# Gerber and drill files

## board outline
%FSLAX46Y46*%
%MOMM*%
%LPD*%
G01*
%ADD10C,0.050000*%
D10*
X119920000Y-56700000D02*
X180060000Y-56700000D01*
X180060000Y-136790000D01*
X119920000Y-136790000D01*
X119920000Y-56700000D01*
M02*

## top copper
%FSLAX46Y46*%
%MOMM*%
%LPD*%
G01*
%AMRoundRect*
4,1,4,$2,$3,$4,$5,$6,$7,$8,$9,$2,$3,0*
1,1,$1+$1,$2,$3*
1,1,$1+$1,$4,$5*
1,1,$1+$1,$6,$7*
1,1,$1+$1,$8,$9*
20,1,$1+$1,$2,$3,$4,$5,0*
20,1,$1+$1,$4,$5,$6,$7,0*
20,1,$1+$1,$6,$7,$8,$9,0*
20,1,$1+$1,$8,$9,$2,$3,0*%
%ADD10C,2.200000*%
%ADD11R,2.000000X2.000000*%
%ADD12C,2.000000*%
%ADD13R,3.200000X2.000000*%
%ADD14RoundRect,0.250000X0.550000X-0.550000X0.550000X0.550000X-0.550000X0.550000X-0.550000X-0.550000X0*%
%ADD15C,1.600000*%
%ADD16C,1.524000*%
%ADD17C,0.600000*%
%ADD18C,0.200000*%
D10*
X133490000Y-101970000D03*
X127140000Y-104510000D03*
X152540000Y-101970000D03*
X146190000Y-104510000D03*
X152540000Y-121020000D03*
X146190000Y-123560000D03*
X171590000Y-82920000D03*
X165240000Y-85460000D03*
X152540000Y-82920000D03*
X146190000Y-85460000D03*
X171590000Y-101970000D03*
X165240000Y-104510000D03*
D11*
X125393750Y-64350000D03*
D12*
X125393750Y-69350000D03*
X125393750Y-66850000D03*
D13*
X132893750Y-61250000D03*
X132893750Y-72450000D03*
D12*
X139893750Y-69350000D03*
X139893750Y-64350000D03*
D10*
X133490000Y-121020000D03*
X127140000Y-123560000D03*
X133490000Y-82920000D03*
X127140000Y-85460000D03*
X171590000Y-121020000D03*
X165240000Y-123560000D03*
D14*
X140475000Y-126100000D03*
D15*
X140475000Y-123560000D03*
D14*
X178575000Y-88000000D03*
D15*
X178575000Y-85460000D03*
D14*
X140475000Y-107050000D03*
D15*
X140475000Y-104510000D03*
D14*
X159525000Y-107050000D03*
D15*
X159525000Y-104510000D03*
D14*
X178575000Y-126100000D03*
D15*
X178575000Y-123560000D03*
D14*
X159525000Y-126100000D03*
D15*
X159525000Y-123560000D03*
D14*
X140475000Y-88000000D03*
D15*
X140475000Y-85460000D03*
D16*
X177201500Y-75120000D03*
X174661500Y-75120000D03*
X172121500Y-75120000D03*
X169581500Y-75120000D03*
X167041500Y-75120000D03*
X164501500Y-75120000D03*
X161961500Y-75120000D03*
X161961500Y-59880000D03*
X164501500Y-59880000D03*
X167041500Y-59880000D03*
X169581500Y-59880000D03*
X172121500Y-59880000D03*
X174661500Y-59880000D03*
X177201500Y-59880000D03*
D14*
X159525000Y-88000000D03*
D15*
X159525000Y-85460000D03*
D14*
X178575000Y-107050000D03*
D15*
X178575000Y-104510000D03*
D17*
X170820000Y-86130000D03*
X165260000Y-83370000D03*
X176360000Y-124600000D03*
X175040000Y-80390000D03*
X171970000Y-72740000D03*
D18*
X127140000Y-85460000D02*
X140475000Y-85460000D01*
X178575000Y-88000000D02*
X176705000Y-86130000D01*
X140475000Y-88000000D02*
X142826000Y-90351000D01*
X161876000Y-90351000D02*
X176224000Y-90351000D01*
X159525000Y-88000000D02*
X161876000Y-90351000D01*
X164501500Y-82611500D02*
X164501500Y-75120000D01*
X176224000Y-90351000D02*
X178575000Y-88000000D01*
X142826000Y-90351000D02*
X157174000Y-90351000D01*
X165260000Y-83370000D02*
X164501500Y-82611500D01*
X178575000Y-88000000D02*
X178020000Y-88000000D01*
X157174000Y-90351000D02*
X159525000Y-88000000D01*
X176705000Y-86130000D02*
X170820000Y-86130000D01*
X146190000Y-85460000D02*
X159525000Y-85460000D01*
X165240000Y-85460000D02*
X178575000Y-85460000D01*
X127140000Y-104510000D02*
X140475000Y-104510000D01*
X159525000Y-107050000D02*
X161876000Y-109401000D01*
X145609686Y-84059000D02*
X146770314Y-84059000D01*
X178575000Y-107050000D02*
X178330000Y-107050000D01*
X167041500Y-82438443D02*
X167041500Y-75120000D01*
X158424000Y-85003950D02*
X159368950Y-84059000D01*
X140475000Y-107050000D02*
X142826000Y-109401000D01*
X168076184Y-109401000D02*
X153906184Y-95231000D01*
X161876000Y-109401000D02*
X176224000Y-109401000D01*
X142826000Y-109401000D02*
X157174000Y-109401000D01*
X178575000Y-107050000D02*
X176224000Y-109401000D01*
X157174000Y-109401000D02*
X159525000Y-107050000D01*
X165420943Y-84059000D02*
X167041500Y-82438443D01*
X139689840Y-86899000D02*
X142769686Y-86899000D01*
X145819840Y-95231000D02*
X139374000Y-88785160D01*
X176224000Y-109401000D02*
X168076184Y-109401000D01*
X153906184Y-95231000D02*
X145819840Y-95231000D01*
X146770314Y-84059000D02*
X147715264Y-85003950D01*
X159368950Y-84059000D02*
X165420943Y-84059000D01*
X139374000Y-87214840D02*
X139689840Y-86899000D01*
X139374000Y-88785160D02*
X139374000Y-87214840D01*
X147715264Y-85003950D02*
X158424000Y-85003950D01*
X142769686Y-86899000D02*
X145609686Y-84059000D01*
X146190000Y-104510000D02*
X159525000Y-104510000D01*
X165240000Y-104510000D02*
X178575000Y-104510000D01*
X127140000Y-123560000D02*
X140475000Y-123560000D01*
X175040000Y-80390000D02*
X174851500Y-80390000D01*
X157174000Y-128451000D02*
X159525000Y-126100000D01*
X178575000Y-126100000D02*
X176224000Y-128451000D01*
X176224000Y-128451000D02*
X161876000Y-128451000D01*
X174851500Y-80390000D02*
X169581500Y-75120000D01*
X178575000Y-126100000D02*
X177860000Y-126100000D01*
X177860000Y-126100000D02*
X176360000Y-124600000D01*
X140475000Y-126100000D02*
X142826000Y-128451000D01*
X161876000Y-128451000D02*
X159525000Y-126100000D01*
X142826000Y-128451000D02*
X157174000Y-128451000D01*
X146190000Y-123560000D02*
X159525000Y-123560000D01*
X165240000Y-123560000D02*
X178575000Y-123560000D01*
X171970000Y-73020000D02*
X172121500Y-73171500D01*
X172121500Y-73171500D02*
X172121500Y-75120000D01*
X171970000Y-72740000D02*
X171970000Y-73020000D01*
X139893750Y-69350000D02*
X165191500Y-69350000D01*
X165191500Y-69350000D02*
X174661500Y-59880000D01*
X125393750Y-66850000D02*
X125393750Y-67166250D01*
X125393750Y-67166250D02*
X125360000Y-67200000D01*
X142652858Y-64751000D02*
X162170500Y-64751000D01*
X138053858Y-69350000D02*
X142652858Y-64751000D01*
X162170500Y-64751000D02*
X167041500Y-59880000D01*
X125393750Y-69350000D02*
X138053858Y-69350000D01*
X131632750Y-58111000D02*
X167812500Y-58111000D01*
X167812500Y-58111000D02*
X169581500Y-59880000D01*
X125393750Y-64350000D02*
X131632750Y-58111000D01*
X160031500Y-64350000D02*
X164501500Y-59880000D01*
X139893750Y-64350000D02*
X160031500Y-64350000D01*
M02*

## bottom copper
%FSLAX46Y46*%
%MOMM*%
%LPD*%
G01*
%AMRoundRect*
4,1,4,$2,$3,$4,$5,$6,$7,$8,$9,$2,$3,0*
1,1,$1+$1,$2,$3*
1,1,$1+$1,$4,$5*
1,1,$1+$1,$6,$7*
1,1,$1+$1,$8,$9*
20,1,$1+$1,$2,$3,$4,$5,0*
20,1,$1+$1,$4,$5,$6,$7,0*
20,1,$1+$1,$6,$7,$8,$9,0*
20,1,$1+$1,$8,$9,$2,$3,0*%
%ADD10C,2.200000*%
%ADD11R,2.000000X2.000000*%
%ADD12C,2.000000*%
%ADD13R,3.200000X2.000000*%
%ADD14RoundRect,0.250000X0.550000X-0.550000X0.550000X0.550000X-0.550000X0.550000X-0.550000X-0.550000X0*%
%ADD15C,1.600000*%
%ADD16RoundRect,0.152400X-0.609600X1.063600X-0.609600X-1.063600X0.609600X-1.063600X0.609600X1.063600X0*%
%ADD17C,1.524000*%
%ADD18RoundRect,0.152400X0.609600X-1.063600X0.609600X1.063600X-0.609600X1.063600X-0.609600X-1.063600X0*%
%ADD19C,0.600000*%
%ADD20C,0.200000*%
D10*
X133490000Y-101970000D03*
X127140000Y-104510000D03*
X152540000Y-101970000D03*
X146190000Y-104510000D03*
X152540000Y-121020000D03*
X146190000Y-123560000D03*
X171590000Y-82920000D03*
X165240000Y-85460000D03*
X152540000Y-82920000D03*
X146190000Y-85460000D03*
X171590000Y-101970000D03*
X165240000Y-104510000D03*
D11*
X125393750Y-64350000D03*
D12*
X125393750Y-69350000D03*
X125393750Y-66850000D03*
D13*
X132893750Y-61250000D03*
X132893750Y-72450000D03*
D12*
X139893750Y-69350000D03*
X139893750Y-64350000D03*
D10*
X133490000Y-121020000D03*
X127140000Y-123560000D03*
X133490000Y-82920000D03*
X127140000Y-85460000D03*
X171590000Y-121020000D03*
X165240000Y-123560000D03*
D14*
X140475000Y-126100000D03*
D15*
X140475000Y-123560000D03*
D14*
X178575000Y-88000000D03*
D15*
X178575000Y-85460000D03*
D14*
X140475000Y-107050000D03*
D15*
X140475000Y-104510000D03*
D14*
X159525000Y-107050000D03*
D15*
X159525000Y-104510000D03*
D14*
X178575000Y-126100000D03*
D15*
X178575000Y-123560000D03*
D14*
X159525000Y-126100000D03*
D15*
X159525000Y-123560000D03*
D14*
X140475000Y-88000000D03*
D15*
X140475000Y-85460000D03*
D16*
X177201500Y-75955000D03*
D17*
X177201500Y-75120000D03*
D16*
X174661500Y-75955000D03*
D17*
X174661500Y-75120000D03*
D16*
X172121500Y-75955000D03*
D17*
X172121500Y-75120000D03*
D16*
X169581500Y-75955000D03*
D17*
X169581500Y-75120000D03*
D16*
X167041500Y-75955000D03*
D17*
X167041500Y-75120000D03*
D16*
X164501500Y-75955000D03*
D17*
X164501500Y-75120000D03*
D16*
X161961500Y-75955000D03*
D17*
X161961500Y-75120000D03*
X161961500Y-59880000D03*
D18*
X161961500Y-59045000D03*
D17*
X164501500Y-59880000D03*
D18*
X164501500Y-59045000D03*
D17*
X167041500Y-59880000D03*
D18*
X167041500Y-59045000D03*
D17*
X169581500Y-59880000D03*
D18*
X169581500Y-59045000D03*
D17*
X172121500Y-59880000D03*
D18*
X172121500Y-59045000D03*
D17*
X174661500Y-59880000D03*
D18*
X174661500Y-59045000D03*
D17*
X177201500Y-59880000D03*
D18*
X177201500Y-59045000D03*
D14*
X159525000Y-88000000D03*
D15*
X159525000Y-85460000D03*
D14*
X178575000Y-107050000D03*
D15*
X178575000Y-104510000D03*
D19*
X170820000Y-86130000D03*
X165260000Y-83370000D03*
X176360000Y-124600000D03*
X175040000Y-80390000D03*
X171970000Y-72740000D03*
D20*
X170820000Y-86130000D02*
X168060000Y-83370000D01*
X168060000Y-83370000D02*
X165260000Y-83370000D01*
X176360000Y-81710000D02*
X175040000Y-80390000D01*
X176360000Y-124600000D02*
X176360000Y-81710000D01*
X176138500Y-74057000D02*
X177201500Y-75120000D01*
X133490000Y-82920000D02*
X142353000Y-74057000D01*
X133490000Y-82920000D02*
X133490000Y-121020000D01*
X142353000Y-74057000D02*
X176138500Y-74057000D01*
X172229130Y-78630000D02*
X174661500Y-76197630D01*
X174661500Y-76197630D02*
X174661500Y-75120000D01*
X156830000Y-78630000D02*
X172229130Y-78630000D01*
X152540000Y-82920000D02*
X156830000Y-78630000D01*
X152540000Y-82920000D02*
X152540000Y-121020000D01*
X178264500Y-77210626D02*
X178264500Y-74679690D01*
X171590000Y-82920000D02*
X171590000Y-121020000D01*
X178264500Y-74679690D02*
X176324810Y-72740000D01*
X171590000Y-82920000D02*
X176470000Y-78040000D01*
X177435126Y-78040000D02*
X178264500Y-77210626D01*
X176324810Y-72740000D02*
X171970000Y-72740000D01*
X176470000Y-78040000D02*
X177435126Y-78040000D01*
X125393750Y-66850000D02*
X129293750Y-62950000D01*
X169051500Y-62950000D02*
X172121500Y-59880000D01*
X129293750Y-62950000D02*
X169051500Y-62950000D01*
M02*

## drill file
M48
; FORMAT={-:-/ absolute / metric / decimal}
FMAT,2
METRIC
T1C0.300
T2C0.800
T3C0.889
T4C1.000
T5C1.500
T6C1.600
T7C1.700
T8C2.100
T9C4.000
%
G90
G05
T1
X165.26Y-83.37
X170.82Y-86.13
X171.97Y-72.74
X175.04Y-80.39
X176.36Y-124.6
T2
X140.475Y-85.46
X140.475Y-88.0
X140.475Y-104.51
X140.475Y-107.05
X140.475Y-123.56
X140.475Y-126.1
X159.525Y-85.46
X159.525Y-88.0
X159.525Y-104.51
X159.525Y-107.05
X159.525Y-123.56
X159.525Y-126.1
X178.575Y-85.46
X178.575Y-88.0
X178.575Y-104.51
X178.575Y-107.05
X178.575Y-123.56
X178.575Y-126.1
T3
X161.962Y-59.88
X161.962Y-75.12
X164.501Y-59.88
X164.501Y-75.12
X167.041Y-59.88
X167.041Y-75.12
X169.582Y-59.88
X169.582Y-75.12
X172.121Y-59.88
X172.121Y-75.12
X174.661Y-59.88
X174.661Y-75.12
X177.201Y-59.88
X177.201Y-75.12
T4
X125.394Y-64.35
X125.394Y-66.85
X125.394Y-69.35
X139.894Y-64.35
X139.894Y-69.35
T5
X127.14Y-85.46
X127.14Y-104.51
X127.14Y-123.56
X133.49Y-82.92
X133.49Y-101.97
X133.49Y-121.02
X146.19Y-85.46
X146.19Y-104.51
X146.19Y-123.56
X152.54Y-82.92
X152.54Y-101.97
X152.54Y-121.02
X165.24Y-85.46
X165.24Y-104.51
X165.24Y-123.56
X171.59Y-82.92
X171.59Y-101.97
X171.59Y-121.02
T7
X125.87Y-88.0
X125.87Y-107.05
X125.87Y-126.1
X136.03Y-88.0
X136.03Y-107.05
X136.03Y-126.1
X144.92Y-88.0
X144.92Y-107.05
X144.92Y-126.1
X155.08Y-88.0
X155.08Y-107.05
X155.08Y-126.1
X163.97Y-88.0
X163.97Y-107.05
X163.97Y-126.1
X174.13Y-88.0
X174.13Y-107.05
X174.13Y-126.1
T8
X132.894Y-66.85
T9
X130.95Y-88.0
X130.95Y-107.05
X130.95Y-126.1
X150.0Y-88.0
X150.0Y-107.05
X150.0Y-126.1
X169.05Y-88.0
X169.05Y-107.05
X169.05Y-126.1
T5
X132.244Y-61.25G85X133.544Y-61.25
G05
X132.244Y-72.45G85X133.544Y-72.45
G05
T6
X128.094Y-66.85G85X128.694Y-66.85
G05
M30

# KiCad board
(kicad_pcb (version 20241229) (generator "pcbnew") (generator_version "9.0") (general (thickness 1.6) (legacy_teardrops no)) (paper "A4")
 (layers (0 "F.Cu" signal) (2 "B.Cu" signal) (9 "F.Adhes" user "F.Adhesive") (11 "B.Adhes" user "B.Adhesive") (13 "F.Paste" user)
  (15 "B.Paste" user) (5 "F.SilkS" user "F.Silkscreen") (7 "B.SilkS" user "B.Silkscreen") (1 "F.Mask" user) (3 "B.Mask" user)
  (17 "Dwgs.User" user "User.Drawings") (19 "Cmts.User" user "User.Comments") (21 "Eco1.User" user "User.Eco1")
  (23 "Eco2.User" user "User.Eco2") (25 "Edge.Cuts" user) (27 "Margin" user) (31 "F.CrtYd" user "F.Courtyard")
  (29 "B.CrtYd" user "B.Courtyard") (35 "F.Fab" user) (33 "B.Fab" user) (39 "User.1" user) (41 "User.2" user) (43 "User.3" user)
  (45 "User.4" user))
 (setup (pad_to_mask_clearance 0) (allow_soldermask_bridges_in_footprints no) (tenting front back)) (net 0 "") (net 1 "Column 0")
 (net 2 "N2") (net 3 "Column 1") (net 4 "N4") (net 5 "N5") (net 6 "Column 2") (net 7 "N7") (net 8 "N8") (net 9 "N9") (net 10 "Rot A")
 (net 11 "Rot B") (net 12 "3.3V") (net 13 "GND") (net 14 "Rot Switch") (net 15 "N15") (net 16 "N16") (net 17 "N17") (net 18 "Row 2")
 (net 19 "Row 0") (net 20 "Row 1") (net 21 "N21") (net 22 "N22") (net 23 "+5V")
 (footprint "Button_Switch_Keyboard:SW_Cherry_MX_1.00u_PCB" (layer "F.Cu") (at 133.49 101.97)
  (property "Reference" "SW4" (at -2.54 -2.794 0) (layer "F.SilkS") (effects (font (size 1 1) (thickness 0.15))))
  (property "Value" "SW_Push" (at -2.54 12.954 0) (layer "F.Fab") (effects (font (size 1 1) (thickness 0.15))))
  (pad "" np_thru_hole circle (at -7.62 5.08) (size 1.7 1.7) (drill 1.7) (layers "*.Cu" "*.Mask"))
  (pad "" np_thru_hole circle (at -2.54 5.08) (size 4 4) (drill 4) (layers "*.Cu" "*.Mask"))
  (pad "" np_thru_hole circle (at 2.54 5.08) (size 1.7 1.7) (drill 1.7) (layers "*.Cu" "*.Mask"))
  (pad "1" thru_hole circle (at 0 0) (size 2.2 2.2) (drill 1.5) (layers "*.Cu" "*.Mask") (remove_unused_layers no) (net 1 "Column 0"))
  (pad "2" thru_hole circle (at -6.35 2.54) (size 2.2 2.2) (drill 1.5) (layers "*.Cu" "*.Mask") (remove_unused_layers no) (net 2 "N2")))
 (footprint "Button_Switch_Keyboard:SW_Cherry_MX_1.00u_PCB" (layer "F.Cu") (at 152.54 101.97)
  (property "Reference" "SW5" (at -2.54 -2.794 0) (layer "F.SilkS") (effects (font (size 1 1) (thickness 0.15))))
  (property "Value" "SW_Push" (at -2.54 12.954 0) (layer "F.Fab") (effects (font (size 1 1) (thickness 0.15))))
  (pad "" np_thru_hole circle (at -7.62 5.08) (size 1.7 1.7) (drill 1.7) (layers "*.Cu" "*.Mask"))
  (pad "" np_thru_hole circle (at -2.54 5.08) (size 4 4) (drill 4) (layers "*.Cu" "*.Mask"))
  (pad "" np_thru_hole circle (at 2.54 5.08) (size 1.7 1.7) (drill 1.7) (layers "*.Cu" "*.Mask"))
  (pad "1" thru_hole circle (at 0 0) (size 2.2 2.2) (drill 1.5) (layers "*.Cu" "*.Mask") (remove_unused_layers no) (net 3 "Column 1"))
  (pad "2" thru_hole circle (at -6.35 2.54) (size 2.2 2.2) (drill 1.5) (layers "*.Cu" "*.Mask") (remove_unused_layers no) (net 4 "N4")))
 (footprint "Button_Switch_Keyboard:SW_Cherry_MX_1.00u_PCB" (layer "F.Cu") (at 152.54 121.02)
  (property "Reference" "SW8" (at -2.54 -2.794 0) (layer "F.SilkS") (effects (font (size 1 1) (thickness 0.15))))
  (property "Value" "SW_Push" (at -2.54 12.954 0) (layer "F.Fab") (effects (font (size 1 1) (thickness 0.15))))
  (pad "" np_thru_hole circle (at -7.62 5.08) (size 1.7 1.7) (drill 1.7) (layers "*.Cu" "*.Mask"))
  (pad "" np_thru_hole circle (at -2.54 5.08) (size 4 4) (drill 4) (layers "*.Cu" "*.Mask"))
  (pad "" np_thru_hole circle (at 2.54 5.08) (size 1.7 1.7) (drill 1.7) (layers "*.Cu" "*.Mask"))
  (pad "1" thru_hole circle (at 0 0) (size 2.2 2.2) (drill 1.5) (layers "*.Cu" "*.Mask") (remove_unused_layers no) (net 3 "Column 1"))
  (pad "2" thru_hole circle (at -6.35 2.54) (size 2.2 2.2) (drill 1.5) (layers "*.Cu" "*.Mask") (remove_unused_layers no) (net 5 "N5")))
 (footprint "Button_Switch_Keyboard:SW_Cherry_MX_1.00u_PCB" (layer "F.Cu") (at 171.59 82.92)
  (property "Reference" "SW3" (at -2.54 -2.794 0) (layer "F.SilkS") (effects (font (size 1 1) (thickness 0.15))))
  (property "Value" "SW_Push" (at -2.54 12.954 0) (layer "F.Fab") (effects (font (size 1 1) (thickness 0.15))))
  (pad "" np_thru_hole circle (at -7.62 5.08) (size 1.7 1.7) (drill 1.7) (layers "*.Cu" "*.Mask"))
  (pad "" np_thru_hole circle (at -2.54 5.08) (size 4 4) (drill 4) (layers "*.Cu" "*.Mask"))
  (pad "" np_thru_hole circle (at 2.54 5.08) (size 1.7 1.7) (drill 1.7) (layers "*.Cu" "*.Mask"))
  (pad "1" thru_hole circle (at 0 0) (size 2.2 2.2) (drill 1.5) (layers "*.Cu" "*.Mask") (remove_unused_layers no) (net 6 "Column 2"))
  (pad "2" thru_hole circle (at -6.35 2.54) (size 2.2 2.2) (drill 1.5) (layers "*.Cu" "*.Mask") (remove_unused_layers no) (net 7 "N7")))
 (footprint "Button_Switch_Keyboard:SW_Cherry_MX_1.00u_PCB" (layer "F.Cu") (at 152.54 82.92)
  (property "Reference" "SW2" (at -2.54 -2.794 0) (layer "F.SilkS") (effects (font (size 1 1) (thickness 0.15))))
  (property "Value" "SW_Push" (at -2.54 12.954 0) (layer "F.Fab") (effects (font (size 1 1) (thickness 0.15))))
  (pad "" np_thru_hole circle (at -7.62 5.08) (size 1.7 1.7) (drill 1.7) (layers "*.Cu" "*.Mask"))
  (pad "" np_thru_hole circle (at -2.54 5.08) (size 4 4) (drill 4) (layers "*.Cu" "*.Mask"))
  (pad "" np_thru_hole circle (at 2.54 5.08) (size 1.7 1.7) (drill 1.7) (layers "*.Cu" "*.Mask"))
  (pad "1" thru_hole circle (at 0 0) (size 2.2 2.2) (drill 1.5) (layers "*.Cu" "*.Mask") (remove_unused_layers no) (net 3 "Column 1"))
  (pad "2" thru_hole circle (at -6.35 2.54) (size 2.2 2.2) (drill 1.5) (layers "*.Cu" "*.Mask") (remove_unused_layers no) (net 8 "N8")))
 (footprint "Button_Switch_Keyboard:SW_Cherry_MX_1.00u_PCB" (layer "F.Cu") (at 171.59 101.97)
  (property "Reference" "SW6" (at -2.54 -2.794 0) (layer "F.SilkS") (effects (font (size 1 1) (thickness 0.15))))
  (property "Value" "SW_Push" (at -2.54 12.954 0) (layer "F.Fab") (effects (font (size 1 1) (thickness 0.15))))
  (pad "" np_thru_hole circle (at -7.62 5.08) (size 1.7 1.7) (drill 1.7) (layers "*.Cu" "*.Mask"))
  (pad "" np_thru_hole circle (at -2.54 5.08) (size 4 4) (drill 4) (layers "*.Cu" "*.Mask"))
  (pad "" np_thru_hole circle (at 2.54 5.08) (size 1.7 1.7) (drill 1.7) (layers "*.Cu" "*.Mask"))
  (pad "1" thru_hole circle (at 0 0) (size 2.2 2.2) (drill 1.5) (layers "*.Cu" "*.Mask") (remove_unused_layers no) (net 6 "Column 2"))
  (pad "2" thru_hole circle (at -6.35 2.54) (size 2.2 2.2) (drill 1.5) (layers "*.Cu" "*.Mask") (remove_unused_layers no) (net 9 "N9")))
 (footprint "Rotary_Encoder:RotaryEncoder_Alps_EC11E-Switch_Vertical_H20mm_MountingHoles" (layer "F.Cu") (at 125.39375 64.35)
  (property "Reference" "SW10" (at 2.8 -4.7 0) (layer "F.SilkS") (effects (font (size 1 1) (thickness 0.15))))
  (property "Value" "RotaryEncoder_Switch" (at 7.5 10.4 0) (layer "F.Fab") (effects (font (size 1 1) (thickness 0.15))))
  (pad "" np_thru_hole oval (at 3 2.5) (size 2.2 1.6) (drill oval 2.2 1.6) (layers "*.Mask"))
  (pad "" np_thru_hole circle (at 7.5 2.5) (size 2.1 2.1) (drill 2.1) (layers "*.Mask"))
  (pad "A" thru_hole rect (at 0 0) (size 2 2) (drill 1) (layers "*.Cu" "*.Mask") (remove_unused_layers no) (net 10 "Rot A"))
  (pad "B" thru_hole circle (at 0 5) (size 2 2) (drill 1) (layers "*.Cu" "*.Mask") (remove_unused_layers no) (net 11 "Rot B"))
  (pad "C" thru_hole circle (at 0 2.5) (size 2 2) (drill 1) (layers "*.Cu" "*.Mask") (remove_unused_layers no) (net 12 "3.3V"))
  (pad "MP" thru_hole rect (at 7.5 -3.1) (size 3.2 2) (drill oval 2.8 1.5) (layers "*.Cu" "*.Mask") (remove_unused_layers no))
  (pad "MP" thru_hole rect (at 7.5 8.1) (size 3.2 2) (drill oval 2.8 1.5) (layers "*.Cu" "*.Mask") (remove_unused_layers no))
  (pad "S1" thru_hole circle (at 14.5 5) (size 2 2) (drill 1) (layers "*.Cu" "*.Mask") (remove_unused_layers no) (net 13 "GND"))
  (pad "S2" thru_hole circle (at 14.5 0) (size 2 2) (drill 1) (layers "*.Cu" "*.Mask") (remove_unused_layers no) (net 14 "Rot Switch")))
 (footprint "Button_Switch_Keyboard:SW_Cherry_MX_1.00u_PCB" (layer "F.Cu") (at 133.49 121.02)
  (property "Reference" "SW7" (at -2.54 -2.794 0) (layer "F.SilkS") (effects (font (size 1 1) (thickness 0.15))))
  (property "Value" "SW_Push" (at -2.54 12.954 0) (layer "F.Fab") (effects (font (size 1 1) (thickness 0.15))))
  (pad "" np_thru_hole circle (at -7.62 5.08) (size 1.7 1.7) (drill 1.7) (layers "*.Cu" "*.Mask"))
  (pad "" np_thru_hole circle (at -2.54 5.08) (size 4 4) (drill 4) (layers "*.Cu" "*.Mask"))
  (pad "" np_thru_hole circle (at 2.54 5.08) (size 1.7 1.7) (drill 1.7) (layers "*.Cu" "*.Mask"))
  (pad "1" thru_hole circle (at 0 0) (size 2.2 2.2) (drill 1.5) (layers "*.Cu" "*.Mask") (remove_unused_layers no) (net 1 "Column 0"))
  (pad "2" thru_hole circle (at -6.35 2.54) (size 2.2 2.2) (drill 1.5) (layers "*.Cu" "*.Mask") (remove_unused_layers no) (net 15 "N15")))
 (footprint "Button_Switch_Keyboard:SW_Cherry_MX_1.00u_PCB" (layer "F.Cu") (at 133.49 82.92)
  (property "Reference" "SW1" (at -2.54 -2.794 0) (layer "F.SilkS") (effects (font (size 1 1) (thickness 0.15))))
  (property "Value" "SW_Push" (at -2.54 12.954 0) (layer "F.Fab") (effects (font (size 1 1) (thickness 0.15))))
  (pad "" np_thru_hole circle (at -7.62 5.08) (size 1.7 1.7) (drill 1.7) (layers "*.Cu" "*.Mask"))
  (pad "" np_thru_hole circle (at -2.54 5.08) (size 4 4) (drill 4) (layers "*.Cu" "*.Mask"))
  (pad "" np_thru_hole circle (at 2.54 5.08) (size 1.7 1.7) (drill 1.7) (layers "*.Cu" "*.Mask"))
  (pad "1" thru_hole circle (at 0 0) (size 2.2 2.2) (drill 1.5) (layers "*.Cu" "*.Mask") (remove_unused_layers no) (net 1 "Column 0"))
  (pad "2" thru_hole circle (at -6.35 2.54) (size 2.2 2.2) (drill 1.5) (layers "*.Cu" "*.Mask") (remove_unused_layers no) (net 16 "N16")))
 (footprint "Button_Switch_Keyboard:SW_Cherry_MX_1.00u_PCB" (layer "F.Cu") (at 171.59 121.02)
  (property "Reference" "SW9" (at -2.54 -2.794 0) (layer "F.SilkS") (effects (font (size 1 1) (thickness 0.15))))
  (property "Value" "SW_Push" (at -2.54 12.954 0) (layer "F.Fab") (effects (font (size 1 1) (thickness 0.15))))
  (pad "" np_thru_hole circle (at -7.62 5.08) (size 1.7 1.7) (drill 1.7) (layers "*.Cu" "*.Mask"))
  (pad "" np_thru_hole circle (at -2.54 5.08) (size 4 4) (drill 4) (layers "*.Cu" "*.Mask"))
  (pad "" np_thru_hole circle (at 2.54 5.08) (size 1.7 1.7) (drill 1.7) (layers "*.Cu" "*.Mask"))
  (pad "1" thru_hole circle (at 0 0) (size 2.2 2.2) (drill 1.5) (layers "*.Cu" "*.Mask") (remove_unused_layers no) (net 6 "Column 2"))
  (pad "2" thru_hole circle (at -6.35 2.54) (size 2.2 2.2) (drill 1.5) (layers "*.Cu" "*.Mask") (remove_unused_layers no) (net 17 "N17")))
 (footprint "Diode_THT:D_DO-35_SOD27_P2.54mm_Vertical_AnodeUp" (layer "B.Cu") (at 140.475 126.1 90)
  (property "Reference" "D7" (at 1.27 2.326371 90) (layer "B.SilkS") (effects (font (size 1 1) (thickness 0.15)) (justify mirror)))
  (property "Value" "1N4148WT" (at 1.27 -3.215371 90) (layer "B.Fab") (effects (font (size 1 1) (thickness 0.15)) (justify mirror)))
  (pad "1" thru_hole roundrect (at 0 0 90) (size 1.6 1.6) (drill 0.8) (layers "*.Cu" "*.Mask") (remove_unused_layers no)
   (roundrect_rratio 0.15625) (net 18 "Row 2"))
  (pad "2" thru_hole circle (at 2.54 0 90) (size 1.6 1.6) (drill 0.8) (layers "*.Cu" "*.Mask") (remove_unused_layers no) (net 15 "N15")))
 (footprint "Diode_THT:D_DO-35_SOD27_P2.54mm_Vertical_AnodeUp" (layer "B.Cu") (at 178.575 88 90)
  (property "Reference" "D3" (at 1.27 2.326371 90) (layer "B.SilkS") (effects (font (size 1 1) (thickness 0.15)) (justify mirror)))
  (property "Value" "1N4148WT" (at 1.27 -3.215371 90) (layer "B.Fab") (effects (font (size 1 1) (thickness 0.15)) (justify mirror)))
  (pad "1" thru_hole roundrect (at 0 0 90) (size 1.6 1.6) (drill 0.8) (layers "*.Cu" "*.Mask") (remove_unused_layers no)
   (roundrect_rratio 0.15625) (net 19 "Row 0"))
  (pad "2" thru_hole circle (at 2.54 0 90) (size 1.6 1.6) (drill 0.8) (layers "*.Cu" "*.Mask") (remove_unused_layers no) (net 7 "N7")))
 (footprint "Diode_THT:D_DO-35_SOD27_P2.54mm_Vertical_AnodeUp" (layer "B.Cu") (at 140.475 107.05 90)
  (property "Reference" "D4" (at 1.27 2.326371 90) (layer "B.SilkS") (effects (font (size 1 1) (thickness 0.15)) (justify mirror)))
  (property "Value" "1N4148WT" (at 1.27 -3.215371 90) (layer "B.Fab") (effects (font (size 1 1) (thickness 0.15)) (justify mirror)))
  (pad "1" thru_hole roundrect (at 0 0 90) (size 1.6 1.6) (drill 0.8) (layers "*.Cu" "*.Mask") (remove_unused_layers no)
   (roundrect_rratio 0.15625) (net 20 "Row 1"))
  (pad "2" thru_hole circle (at 2.54 0 90) (size 1.6 1.6) (drill 0.8) (layers "*.Cu" "*.Mask") (remove_unused_layers no) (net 2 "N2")))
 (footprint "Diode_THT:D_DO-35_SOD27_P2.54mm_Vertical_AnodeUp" (layer "B.Cu") (at 159.525 107.05 90)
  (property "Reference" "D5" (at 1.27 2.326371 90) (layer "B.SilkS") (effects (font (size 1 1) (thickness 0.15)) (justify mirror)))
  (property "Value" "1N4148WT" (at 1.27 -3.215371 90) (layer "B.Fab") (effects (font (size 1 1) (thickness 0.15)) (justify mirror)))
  (pad "1" thru_hole roundrect (at 0 0 90) (size 1.6 1.6) (drill 0.8) (layers "*.Cu" "*.Mask") (remove_unused_layers no)
   (roundrect_rratio 0.15625) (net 20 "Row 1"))
  (pad "2" thru_hole circle (at 2.54 0 90) (size 1.6 1.6) (drill 0.8) (layers "*.Cu" "*.Mask") (remove_unused_layers no) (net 4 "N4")))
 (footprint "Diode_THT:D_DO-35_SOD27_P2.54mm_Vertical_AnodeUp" (layer "B.Cu") (at 178.575 126.1 90)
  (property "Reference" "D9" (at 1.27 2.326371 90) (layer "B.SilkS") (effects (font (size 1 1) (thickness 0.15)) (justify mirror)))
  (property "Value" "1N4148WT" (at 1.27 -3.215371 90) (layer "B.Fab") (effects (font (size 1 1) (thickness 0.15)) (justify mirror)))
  (pad "1" thru_hole roundrect (at 0 0 90) (size 1.6 1.6) (drill 0.8) (layers "*.Cu" "*.Mask") (remove_unused_layers no)
   (roundrect_rratio 0.15625) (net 18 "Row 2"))
  (pad "2" thru_hole circle (at 2.54 0 90) (size 1.6 1.6) (drill 0.8) (layers "*.Cu" "*.Mask") (remove_unused_layers no) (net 17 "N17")))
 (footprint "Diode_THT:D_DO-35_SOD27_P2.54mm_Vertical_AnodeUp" (layer "B.Cu") (at 159.525 126.1 90)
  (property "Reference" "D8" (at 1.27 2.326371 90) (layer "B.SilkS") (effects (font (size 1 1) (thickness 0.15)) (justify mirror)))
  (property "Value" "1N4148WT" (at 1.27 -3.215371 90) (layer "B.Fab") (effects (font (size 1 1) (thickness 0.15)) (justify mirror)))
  (pad "1" thru_hole roundrect (at 0 0 90) (size 1.6 1.6) (drill 0.8) (layers "*.Cu" "*.Mask") (remove_unused_layers no)
   (roundrect_rratio 0.15625) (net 18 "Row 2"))
  (pad "2" thru_hole circle (at 2.54 0 90) (size 1.6 1.6) (drill 0.8) (layers "*.Cu" "*.Mask") (remove_unused_layers no) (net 5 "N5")))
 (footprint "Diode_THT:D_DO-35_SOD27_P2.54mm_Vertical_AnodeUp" (layer "B.Cu") (at 140.475 88 90)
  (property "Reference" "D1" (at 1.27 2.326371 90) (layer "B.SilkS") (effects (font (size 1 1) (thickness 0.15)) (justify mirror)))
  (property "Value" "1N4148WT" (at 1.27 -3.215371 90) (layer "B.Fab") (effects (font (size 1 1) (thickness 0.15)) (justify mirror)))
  (pad "1" thru_hole roundrect (at 0 0 90) (size 1.6 1.6) (drill 0.8) (layers "*.Cu" "*.Mask") (remove_unused_layers no)
   (roundrect_rratio 0.15625) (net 19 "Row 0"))
  (pad "2" thru_hole circle (at 2.54 0 90) (size 1.6 1.6) (drill 0.8) (layers "*.Cu" "*.Mask") (remove_unused_layers no) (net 16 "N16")))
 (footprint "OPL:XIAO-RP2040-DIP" (layer "B.Cu") (at 169.5815 67.5 90)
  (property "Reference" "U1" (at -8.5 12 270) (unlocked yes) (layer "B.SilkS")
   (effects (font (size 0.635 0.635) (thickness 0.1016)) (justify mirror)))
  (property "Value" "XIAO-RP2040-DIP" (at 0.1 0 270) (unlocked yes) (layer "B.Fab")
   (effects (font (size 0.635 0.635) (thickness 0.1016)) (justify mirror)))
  (pad "1" smd roundrect (at -8.455 7.62 270) (size 2.432 1.524) (layers "B.Cu" "B.Mask") (roundrect_rratio 0.1) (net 1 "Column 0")
   (thermal_bridge_angle 45))
  (pad "1" thru_hole circle (at -7.62 7.62 270) (size 1.524 1.524) (drill 0.889) (layers "*.Cu" "*.Mask") (remove_unused_layers no)
   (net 1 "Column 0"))
  (pad "2" smd roundrect (at -8.455 5.08 270) (size 2.432 1.524) (layers "B.Cu" "B.Mask") (roundrect_rratio 0.1) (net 3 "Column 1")
   (thermal_bridge_angle 45))
  (pad "2" thru_hole circle (at -7.62 5.08 270) (size 1.524 1.524) (drill 0.889) (layers "*.Cu" "*.Mask") (remove_unused_layers no)
   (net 3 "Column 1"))
  (pad "3" smd roundrect (at -8.455 2.54 270) (size 2.432 1.524) (layers "B.Cu" "B.Mask") (roundrect_rratio 0.1) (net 6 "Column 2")
   (thermal_bridge_angle 45))
  (pad "3" thru_hole circle (at -7.62 2.54 270) (size 1.524 1.524) (drill 0.889) (layers "*.Cu" "*.Mask") (remove_unused_layers no)
   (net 6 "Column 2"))
  (pad "4" smd roundrect (at -8.455 0 270) (size 2.432 1.524) (layers "B.Cu" "B.Mask") (roundrect_rratio 0.1) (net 18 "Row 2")
   (thermal_bridge_angle 45))
  (pad "4" thru_hole circle (at -7.62 0 270) (size 1.524 1.524) (drill 0.889) (layers "*.Cu" "*.Mask") (remove_unused_layers no)
   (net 18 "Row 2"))
  (pad "5" smd roundrect (at -8.455 -2.54 270) (size 2.432 1.524) (layers "B.Cu" "B.Mask") (roundrect_rratio 0.1) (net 20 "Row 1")
   (thermal_bridge_angle 45))
  (pad "5" thru_hole circle (at -7.62 -2.54 270) (size 1.524 1.524) (drill 0.889) (layers "*.Cu" "*.Mask") (remove_unused_layers no)
   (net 20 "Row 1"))
  (pad "6" smd roundrect (at -8.455 -5.08 270) (size 2.432 1.524) (layers "B.Cu" "B.Mask") (roundrect_rratio 0.1) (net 19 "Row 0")
   (thermal_bridge_angle 45))
  (pad "6" thru_hole circle (at -7.62 -5.08 270) (size 1.524 1.524) (drill 0.889) (layers "*.Cu" "*.Mask") (remove_unused_layers no)
   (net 19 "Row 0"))
  (pad "7" smd roundrect (at -8.455 -7.62 270) (size 2.432 1.524) (layers "B.Cu" "B.Mask") (roundrect_rratio 0.1) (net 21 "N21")
   (thermal_bridge_angle 45))
  (pad "7" thru_hole circle (at -7.62 -7.62 270) (size 1.524 1.524) (drill 0.889) (layers "*.Cu" "*.Mask") (remove_unused_layers no)
   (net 21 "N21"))
  (pad "8" thru_hole circle (at 7.62 -7.62 90) (size 1.524 1.524) (drill 0.889) (layers "*.Cu" "*.Mask") (remove_unused_layers no)
   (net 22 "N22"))
  (pad "8" smd roundrect (at 8.455 -7.62 90) (size 2.432 1.524) (layers "B.Cu" "B.Mask") (roundrect_rratio 0.1) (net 22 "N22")
   (thermal_bridge_angle 45))
  (pad "9" thru_hole circle (at 7.62 -5.08 90) (size 1.524 1.524) (drill 0.889) (layers "*.Cu" "*.Mask") (remove_unused_layers no)
   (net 14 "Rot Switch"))
  (pad "9" smd roundrect (at 8.455 -5.08 90) (size 2.432 1.524) (layers "B.Cu" "B.Mask") (roundrect_rratio 0.1) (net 14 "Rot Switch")
   (thermal_bridge_angle 45))
  (pad "10" thru_hole circle (at 7.62 -2.54 90) (size 1.524 1.524) (drill 0.889) (layers "*.Cu" "*.Mask") (remove_unused_layers no)
   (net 11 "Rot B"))
  (pad "10" smd roundrect (at 8.455 -2.54 90) (size 2.432 1.524) (layers "B.Cu" "B.Mask") (roundrect_rratio 0.1) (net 11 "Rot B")
   (thermal_bridge_angle 45))
  (pad "11" thru_hole circle (at 7.62 0 90) (size 1.524 1.524) (drill 0.889) (layers "*.Cu" "*.Mask") (remove_unused_layers no)
   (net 10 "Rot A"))
  (pad "11" smd roundrect (at 8.455 0 90) (size 2.432 1.524) (layers "B.Cu" "B.Mask") (roundrect_rratio 0.1) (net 10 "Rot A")
   (thermal_bridge_angle 45))
  (pad "12" thru_hole circle (at 7.62 2.54 90) (size 1.524 1.524) (drill 0.889) (layers "*.Cu" "*.Mask") (remove_unused_layers no)
   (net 12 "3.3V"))
  (pad "12" smd roundrect (at 8.455 2.54 90) (size 2.432 1.524) (layers "B.Cu" "B.Mask") (roundrect_rratio 0.1) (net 12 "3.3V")
   (thermal_bridge_angle 45))
  (pad "13" thru_hole circle (at 7.62 5.08 90) (size 1.524 1.524) (drill 0.889) (layers "*.Cu" "*.Mask") (remove_unused_layers no)
   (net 13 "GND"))
  (pad "13" smd roundrect (at 8.455 5.08 90) (size 2.432 1.524) (layers "B.Cu" "B.Mask") (roundrect_rratio 0.1) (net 13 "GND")
   (thermal_bridge_angle 45))
  (pad "14" thru_hole circle (at 7.62 7.62 90) (size 1.524 1.524) (drill 0.889) (layers "*.Cu" "*.Mask") (remove_unused_layers no)
   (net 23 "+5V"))
  (pad "14" smd roundrect (at 8.455 7.62 90) (size 2.432 1.524) (layers "B.Cu" "B.Mask") (roundrect_rratio 0.1) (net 23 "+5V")
   (thermal_bridge_angle 45)))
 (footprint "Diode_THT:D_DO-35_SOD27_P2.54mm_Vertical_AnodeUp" (layer "B.Cu") (at 159.525 88 90)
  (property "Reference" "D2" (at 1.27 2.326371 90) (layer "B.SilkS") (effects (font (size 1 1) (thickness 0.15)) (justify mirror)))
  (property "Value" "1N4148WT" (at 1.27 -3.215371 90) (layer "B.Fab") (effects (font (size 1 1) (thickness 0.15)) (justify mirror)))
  (pad "1" thru_hole roundrect (at 0 0 90) (size 1.6 1.6) (drill 0.8) (layers "*.Cu" "*.Mask") (remove_unused_layers no)
   (roundrect_rratio 0.15625) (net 19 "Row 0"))
  (pad "2" thru_hole circle (at 2.54 0 90) (size 1.6 1.6) (drill 0.8) (layers "*.Cu" "*.Mask") (remove_unused_layers no) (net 8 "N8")))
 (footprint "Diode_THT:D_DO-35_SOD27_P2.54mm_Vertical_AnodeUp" (layer "B.Cu") (at 178.575 107.05 90)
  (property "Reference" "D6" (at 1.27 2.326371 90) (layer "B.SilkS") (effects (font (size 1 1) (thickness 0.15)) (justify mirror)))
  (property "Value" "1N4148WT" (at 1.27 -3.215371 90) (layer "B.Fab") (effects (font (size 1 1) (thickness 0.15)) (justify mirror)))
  (pad "1" thru_hole roundrect (at 0 0 90) (size 1.6 1.6) (drill 0.8) (layers "*.Cu" "*.Mask") (remove_unused_layers no)
   (roundrect_rratio 0.15625) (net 20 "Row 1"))
  (pad "2" thru_hole circle (at 2.54 0 90) (size 1.6 1.6) (drill 0.8) (layers "*.Cu" "*.Mask") (remove_unused_layers no) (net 9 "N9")))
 (gr_rect (start 119.92 56.7) (end 180.06 136.79) (stroke (width 0.05) (type default)) (fill no) (layer "Edge.Cuts"))
 (segment (start 127.14 85.46) (end 140.475 85.46) (width 0.2) (layer "F.Cu") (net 16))
 (segment (start 178.575 88) (end 176.705 86.13) (width 0.2) (layer "F.Cu") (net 19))
 (segment (start 140.475 88) (end 142.826 90.351) (width 0.2) (layer "F.Cu") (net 19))
 (segment (start 161.876 90.351) (end 176.224 90.351) (width 0.2) (layer "F.Cu") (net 19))
 (segment (start 159.525 88) (end 161.876 90.351) (width 0.2) (layer "F.Cu") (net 19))
 (segment (start 164.5015 82.6115) (end 164.5015 75.12) (width 0.2) (layer "F.Cu") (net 19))
 (segment (start 176.224 90.351) (end 178.575 88) (width 0.2) (layer "F.Cu") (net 19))
 (segment (start 142.826 90.351) (end 157.174 90.351) (width 0.2) (layer "F.Cu") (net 19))
 (segment (start 165.26 83.37) (end 164.5015 82.6115) (width 0.2) (layer "F.Cu") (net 19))
 (segment (start 178.575 88) (end 178.02 88) (width 0.2) (layer "F.Cu") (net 19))
 (segment (start 157.174 90.351) (end 159.525 88) (width 0.2) (layer "F.Cu") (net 19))
 (segment (start 176.705 86.13) (end 170.82 86.13) (width 0.2) (layer "F.Cu") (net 19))
 (via (at 170.82 86.13) (size 0.6) (drill 0.3) (layers "F.Cu" "B.Cu") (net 19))
 (via (at 165.26 83.37) (size 0.6) (drill 0.3) (layers "F.Cu" "B.Cu") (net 19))
 (segment (start 170.82 86.13) (end 168.06 83.37) (width 0.2) (layer "B.Cu") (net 19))
 (segment (start 168.06 83.37) (end 165.26 83.37) (width 0.2) (layer "B.Cu") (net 19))
 (segment (start 146.19 85.46) (end 159.525 85.46) (width 0.2) (layer "F.Cu") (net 8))
 (segment (start 165.24 85.46) (end 178.575 85.46) (width 0.2) (layer "F.Cu") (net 7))
 (segment (start 127.14 104.51) (end 140.475 104.51) (width 0.2) (layer "F.Cu") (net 2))
 (segment (start 159.525 107.05) (end 161.876 109.401) (width 0.2) (layer "F.Cu") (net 20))
 (segment (start 145.609686 84.059) (end 146.770314 84.059) (width 0.2) (layer "F.Cu") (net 20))
 (segment (start 178.575 107.05) (end 178.33 107.05) (width 0.2) (layer "F.Cu") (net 20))
 (segment (start 167.0415 82.438443) (end 167.0415 75.12) (width 0.2) (layer "F.Cu") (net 20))
 (segment (start 158.424 85.00395) (end 159.36895 84.059) (width 0.2) (layer "F.Cu") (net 20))
 (segment (start 140.475 107.05) (end 142.826 109.401) (width 0.2) (layer "F.Cu") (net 20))
 (segment (start 168.076184 109.401) (end 153.906184 95.231) (width 0.2) (layer "F.Cu") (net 20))
 (segment (start 161.876 109.401) (end 176.224 109.401) (width 0.2) (layer "F.Cu") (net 20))
 (segment (start 142.826 109.401) (end 157.174 109.401) (width 0.2) (layer "F.Cu") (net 20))
 (segment (start 178.575 107.05) (end 176.224 109.401) (width 0.2) (layer "F.Cu") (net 20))
 (segment (start 157.174 109.401) (end 159.525 107.05) (width 0.2) (layer "F.Cu") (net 20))
 (segment (start 165.420943 84.059) (end 167.0415 82.438443) (width 0.2) (layer "F.Cu") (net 20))
 (segment (start 139.68984 86.899) (end 142.769686 86.899) (width 0.2) (layer "F.Cu") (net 20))
 (segment (start 145.81984 95.231) (end 139.374 88.78516) (width 0.2) (layer "F.Cu") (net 20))
 (segment (start 176.224 109.401) (end 168.076184 109.401) (width 0.2) (layer "F.Cu") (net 20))
 (segment (start 153.906184 95.231) (end 145.81984 95.231) (width 0.2) (layer "F.Cu") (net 20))
 (segment (start 146.770314 84.059) (end 147.715264 85.00395) (width 0.2) (layer "F.Cu") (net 20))
 (segment (start 159.36895 84.059) (end 165.420943 84.059) (width 0.2) (layer "F.Cu") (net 20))
 (segment (start 139.374 87.21484) (end 139.68984 86.899) (width 0.2) (layer "F.Cu") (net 20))
 (segment (start 139.374 88.78516) (end 139.374 87.21484) (width 0.2) (layer "F.Cu") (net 20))
 (segment (start 147.715264 85.00395) (end 158.424 85.00395) (width 0.2) (layer "F.Cu") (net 20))
 (segment (start 142.769686 86.899) (end 145.609686 84.059) (width 0.2) (layer "F.Cu") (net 20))
 (segment (start 146.19 104.51) (end 159.525 104.51) (width 0.2) (layer "F.Cu") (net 4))
 (segment (start 165.24 104.51) (end 178.575 104.51) (width 0.2) (layer "F.Cu") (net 9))
 (segment (start 127.14 123.56) (end 140.475 123.56) (width 0.2) (layer "F.Cu") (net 15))
 (segment (start 175.04 80.39) (end 174.8515 80.39) (width 0.2) (layer "F.Cu") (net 18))
 (segment (start 157.174 128.451) (end 159.525 126.1) (width 0.2) (layer "F.Cu") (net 18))
 (segment (start 178.575 126.1) (end 176.224 128.451) (width 0.2) (layer "F.Cu") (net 18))
 (segment (start 176.224 128.451) (end 161.876 128.451) (width 0.2) (layer "F.Cu") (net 18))
 (segment (start 174.8515 80.39) (end 169.5815 75.12) (width 0.2) (layer "F.Cu") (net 18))
 (segment (start 178.575 126.1) (end 177.86 126.1) (width 0.2) (layer "F.Cu") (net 18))
 (segment (start 177.86 126.1) (end 176.36 124.6) (width 0.2) (layer "F.Cu") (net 18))
 (segment (start 140.475 126.1) (end 142.826 128.451) (width 0.2) (layer "F.Cu") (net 18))
 (segment (start 161.876 128.451) (end 159.525 126.1) (width 0.2) (layer "F.Cu") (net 18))
 (segment (start 142.826 128.451) (end 157.174 128.451) (width 0.2) (layer "F.Cu") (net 18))
 (via (at 176.36 124.6) (size 0.6) (drill 0.3) (layers "F.Cu" "B.Cu") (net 18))
 (via (at 175.04 80.39) (size 0.6) (drill 0.3) (layers "F.Cu" "B.Cu") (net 18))
 (segment (start 176.36 81.71) (end 175.04 80.39) (width 0.2) (layer "B.Cu") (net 18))
 (segment (start 176.36 124.6) (end 176.36 81.71) (width 0.2) (layer "B.Cu") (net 18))
 (segment (start 146.19 123.56) (end 159.525 123.56) (width 0.2) (layer "F.Cu") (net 5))
 (segment (start 165.24 123.56) (end 178.575 123.56) (width 0.2) (layer "F.Cu") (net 17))
 (segment (start 176.1385 74.057) (end 177.2015 75.12) (width 0.2) (layer "B.Cu") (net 1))
 (segment (start 133.49 82.92) (end 142.353 74.057) (width 0.2) (layer "B.Cu") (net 1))
 (segment (start 133.49 82.92) (end 133.49 121.02) (width 0.2) (layer "B.Cu") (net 1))
 (segment (start 142.353 74.057) (end 176.1385 74.057) (width 0.2) (layer "B.Cu") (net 1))
 (segment (start 172.22913 78.63) (end 174.6615 76.19763) (width 0.2) (layer "B.Cu") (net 3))
 (segment (start 174.6615 76.19763) (end 174.6615 75.12) (width 0.2) (layer "B.Cu") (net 3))
 (segment (start 156.83 78.63) (end 172.22913 78.63) (width 0.2) (layer "B.Cu") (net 3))
 (segment (start 152.54 82.92) (end 156.83 78.63) (width 0.2) (layer "B.Cu") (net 3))
 (segment (start 152.54 82.92) (end 152.54 121.02) (width 0.2) (layer "B.Cu") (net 3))
 (segment (start 171.97 73.02) (end 172.1215 73.1715) (width 0.2) (layer "F.Cu") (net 6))
 (segment (start 172.1215 73.1715) (end 172.1215 75.12) (width 0.2) (layer "F.Cu") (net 6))
 (segment (start 171.97 72.74) (end 171.97 73.02) (width 0.2) (layer "F.Cu") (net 6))
 (via (at 171.97 72.74) (size 0.6) (drill 0.3) (layers "F.Cu" "B.Cu") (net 6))
 (segment (start 178.2645 77.210626) (end 178.2645 74.67969) (width 0.2) (layer "B.Cu") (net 6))
 (segment (start 171.59 82.92) (end 171.59 121.02) (width 0.2) (layer "B.Cu") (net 6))
 (segment (start 178.2645 74.67969) (end 176.32481 72.74) (width 0.2) (layer "B.Cu") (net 6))
 (segment (start 171.59 82.92) (end 176.47 78.04) (width 0.2) (layer "B.Cu") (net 6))
 (segment (start 177.435126 78.04) (end 178.2645 77.210626) (width 0.2) (layer "B.Cu") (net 6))
 (segment (start 176.32481 72.74) (end 171.97 72.74) (width 0.2) (layer "B.Cu") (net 6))
 (segment (start 176.47 78.04) (end 177.435126 78.04) (width 0.2) (layer "B.Cu") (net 6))
 (segment (start 139.89375 69.35) (end 165.1915 69.35) (width 0.2) (layer "F.Cu") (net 13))
 (segment (start 165.1915 69.35) (end 174.6615 59.88) (width 0.2) (layer "F.Cu") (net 13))
 (segment (start 125.39375 66.85) (end 125.39375 67.16625) (width 0.2) (layer "F.Cu") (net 12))
 (segment (start 125.39375 67.16625) (end 125.36 67.2) (width 0.2) (layer "F.Cu") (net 12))
 (segment (start 125.39375 66.85) (end 129.29375 62.95) (width 0.2) (layer "B.Cu") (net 12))
 (segment (start 169.0515 62.95) (end 172.1215 59.88) (width 0.2) (layer "B.Cu") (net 12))
 (segment (start 129.29375 62.95) (end 169.0515 62.95) (width 0.2) (layer "B.Cu") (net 12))
 (segment (start 142.652858 64.751) (end 162.1705 64.751) (width 0.2) (layer "F.Cu") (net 11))
 (segment (start 138.053858 69.35) (end 142.652858 64.751) (width 0.2) (layer "F.Cu") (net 11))
 (segment (start 162.1705 64.751) (end 167.0415 59.88) (width 0.2) (layer "F.Cu") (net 11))
 (segment (start 125.39375 69.35) (end 138.053858 69.35) (width 0.2) (layer "F.Cu") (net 11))
 (segment (start 131.63275 58.111) (end 167.8125 58.111) (width 0.2) (layer "F.Cu") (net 10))
 (segment (start 167.8125 58.111) (end 169.5815 59.88) (width 0.2) (layer "F.Cu") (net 10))
 (segment (start 125.39375 64.35) (end 131.63275 58.111) (width 0.2) (layer "F.Cu") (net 10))
 (segment (start 160.0315 64.35) (end 164.5015 59.88) (width 0.2) (layer "F.Cu") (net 14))
 (segment (start 139.89375 64.35) (end 160.0315 64.35) (width 0.2) (layer "F.Cu") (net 14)))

